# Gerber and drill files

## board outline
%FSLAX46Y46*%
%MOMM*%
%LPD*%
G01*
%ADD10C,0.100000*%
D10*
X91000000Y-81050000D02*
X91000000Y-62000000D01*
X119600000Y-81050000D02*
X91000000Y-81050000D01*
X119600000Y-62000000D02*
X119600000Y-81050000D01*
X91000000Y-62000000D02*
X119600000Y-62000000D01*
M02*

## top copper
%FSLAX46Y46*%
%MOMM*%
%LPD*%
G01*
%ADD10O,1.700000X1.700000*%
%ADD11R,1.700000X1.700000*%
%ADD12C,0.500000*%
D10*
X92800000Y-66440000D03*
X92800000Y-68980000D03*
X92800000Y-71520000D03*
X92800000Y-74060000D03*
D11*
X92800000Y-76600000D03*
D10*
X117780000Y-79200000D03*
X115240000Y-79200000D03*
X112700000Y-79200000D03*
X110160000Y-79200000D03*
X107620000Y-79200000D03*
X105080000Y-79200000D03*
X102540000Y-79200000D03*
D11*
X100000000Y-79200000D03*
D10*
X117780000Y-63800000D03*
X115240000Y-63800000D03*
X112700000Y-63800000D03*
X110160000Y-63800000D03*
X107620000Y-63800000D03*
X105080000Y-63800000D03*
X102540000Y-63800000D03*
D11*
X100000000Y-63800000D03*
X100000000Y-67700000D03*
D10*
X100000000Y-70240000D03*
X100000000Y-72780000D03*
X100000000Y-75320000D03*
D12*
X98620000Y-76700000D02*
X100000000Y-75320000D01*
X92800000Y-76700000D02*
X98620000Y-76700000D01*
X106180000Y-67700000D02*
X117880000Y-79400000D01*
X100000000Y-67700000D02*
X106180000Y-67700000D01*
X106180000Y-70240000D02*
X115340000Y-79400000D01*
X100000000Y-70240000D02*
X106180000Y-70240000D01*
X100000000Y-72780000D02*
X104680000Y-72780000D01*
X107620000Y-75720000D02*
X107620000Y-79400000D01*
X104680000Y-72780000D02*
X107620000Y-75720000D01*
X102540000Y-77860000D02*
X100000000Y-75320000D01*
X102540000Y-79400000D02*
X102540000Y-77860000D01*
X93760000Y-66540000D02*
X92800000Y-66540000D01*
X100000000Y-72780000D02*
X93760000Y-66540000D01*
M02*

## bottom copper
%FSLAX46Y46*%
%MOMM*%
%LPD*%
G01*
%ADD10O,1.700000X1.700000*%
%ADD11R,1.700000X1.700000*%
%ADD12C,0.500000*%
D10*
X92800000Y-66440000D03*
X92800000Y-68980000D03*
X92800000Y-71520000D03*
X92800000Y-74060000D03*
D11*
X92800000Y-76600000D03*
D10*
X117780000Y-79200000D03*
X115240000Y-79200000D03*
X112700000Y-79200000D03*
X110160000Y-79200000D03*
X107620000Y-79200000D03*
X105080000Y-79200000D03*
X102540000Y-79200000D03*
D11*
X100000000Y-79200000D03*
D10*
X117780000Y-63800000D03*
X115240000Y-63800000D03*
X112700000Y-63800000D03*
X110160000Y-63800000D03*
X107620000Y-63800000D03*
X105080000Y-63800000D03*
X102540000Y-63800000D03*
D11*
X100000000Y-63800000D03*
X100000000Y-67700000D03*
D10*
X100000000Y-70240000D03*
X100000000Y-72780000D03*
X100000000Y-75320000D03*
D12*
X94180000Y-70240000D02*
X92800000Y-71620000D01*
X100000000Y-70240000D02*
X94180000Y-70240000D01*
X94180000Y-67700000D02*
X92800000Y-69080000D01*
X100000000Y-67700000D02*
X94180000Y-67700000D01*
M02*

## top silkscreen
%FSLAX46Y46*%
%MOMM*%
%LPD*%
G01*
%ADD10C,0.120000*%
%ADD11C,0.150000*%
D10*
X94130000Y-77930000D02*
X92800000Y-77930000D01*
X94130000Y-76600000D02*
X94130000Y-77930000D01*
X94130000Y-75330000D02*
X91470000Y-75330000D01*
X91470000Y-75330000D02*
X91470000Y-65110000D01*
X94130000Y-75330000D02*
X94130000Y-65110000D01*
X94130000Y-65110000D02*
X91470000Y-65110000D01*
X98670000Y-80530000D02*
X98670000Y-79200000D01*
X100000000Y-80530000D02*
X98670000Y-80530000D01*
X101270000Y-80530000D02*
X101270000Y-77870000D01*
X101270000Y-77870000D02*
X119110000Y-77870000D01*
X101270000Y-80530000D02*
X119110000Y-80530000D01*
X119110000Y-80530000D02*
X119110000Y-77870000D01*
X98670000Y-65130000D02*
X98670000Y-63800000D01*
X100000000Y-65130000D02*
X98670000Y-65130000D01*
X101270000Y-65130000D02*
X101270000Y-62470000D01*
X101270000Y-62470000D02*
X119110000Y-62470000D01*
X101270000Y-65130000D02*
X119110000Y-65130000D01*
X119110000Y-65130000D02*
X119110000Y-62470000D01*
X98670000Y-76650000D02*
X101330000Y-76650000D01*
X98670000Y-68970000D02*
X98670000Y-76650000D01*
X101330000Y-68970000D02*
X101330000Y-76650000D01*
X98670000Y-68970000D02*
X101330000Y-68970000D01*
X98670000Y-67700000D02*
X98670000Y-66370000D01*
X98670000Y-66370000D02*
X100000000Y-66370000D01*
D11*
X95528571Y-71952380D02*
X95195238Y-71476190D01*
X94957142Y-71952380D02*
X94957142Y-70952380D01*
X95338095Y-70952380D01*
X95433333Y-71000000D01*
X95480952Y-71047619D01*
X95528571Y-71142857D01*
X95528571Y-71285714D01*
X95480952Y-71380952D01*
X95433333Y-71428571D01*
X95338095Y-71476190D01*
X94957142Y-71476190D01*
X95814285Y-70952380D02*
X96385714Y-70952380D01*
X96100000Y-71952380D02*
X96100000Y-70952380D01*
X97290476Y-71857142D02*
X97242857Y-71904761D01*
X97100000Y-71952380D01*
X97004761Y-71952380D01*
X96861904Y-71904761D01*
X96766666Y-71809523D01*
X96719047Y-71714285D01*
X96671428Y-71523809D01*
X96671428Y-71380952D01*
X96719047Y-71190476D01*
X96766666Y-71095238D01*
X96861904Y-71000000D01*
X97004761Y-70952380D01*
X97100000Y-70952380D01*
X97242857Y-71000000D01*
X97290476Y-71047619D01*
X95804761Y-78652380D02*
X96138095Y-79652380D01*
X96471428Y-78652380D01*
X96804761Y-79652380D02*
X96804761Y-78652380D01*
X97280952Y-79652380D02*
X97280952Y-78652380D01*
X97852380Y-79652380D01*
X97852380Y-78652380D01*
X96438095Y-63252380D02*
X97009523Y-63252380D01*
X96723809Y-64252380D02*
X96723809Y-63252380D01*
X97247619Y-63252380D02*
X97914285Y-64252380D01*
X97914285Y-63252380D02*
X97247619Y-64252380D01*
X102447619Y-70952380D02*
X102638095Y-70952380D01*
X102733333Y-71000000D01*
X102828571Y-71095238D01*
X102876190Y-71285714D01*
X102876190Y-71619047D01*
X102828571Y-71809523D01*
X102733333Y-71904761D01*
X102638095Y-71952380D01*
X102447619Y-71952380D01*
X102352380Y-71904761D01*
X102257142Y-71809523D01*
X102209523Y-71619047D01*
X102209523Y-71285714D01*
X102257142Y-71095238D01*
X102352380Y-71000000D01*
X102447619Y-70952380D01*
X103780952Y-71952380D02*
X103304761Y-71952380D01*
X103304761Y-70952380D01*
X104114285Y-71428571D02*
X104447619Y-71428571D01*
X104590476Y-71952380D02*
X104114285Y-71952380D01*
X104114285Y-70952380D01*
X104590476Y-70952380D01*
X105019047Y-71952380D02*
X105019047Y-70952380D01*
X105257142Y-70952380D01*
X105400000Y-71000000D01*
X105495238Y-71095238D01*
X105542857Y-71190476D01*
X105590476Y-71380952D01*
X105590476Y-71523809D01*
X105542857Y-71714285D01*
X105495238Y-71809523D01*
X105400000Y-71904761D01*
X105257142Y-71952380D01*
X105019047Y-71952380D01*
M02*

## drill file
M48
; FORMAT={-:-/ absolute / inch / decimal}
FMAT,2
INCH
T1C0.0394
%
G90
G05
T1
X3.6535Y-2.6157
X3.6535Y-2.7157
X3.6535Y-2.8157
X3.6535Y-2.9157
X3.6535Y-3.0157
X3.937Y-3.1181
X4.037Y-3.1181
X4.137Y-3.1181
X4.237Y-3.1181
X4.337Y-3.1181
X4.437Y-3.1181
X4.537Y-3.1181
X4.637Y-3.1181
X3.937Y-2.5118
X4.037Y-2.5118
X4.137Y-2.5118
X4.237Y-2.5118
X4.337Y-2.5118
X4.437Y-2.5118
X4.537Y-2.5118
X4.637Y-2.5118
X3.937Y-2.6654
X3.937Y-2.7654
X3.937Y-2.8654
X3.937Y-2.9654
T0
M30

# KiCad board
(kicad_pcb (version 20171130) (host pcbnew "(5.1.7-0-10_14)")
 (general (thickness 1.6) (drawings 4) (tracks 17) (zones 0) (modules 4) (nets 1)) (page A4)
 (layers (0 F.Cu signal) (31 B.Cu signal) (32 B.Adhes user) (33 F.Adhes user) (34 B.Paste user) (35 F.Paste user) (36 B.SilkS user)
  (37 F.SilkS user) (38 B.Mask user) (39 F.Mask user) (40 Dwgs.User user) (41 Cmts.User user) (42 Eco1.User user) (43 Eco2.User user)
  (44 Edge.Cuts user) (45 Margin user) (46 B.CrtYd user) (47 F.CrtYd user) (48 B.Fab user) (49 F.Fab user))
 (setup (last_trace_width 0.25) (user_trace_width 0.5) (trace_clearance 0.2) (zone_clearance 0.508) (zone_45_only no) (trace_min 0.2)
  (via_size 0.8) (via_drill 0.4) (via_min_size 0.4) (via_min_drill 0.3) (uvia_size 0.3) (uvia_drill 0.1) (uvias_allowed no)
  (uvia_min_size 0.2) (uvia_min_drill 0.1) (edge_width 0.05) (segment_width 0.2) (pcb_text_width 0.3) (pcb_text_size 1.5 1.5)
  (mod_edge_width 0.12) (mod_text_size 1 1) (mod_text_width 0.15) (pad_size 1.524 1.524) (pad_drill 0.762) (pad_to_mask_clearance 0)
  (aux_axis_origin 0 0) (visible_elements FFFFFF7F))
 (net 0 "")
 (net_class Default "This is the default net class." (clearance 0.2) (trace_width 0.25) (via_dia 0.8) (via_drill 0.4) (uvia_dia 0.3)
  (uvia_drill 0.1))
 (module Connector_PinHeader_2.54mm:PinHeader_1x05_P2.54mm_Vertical (layer F.Cu) (at 92.8 76.6 180)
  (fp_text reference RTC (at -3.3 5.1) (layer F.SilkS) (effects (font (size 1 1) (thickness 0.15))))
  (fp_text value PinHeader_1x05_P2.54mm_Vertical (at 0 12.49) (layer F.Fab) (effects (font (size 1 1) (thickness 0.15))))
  (fp_line (start -1.33 -1.33) (end 0 -1.33) (layer F.SilkS) (width 0.12))
  (fp_line (start -1.33 0) (end -1.33 -1.33) (layer F.SilkS) (width 0.12))
  (fp_line (start -1.33 1.27) (end 1.33 1.27) (layer F.SilkS) (width 0.12))
  (fp_line (start 1.33 1.27) (end 1.33 11.49) (layer F.SilkS) (width 0.12))
  (fp_line (start -1.33 1.27) (end -1.33 11.49) (layer F.SilkS) (width 0.12))
  (fp_line (start -1.33 11.49) (end 1.33 11.49) (layer F.SilkS) (width 0.12))
  (pad 5 thru_hole oval (at 0 10.16 180) (size 1.7 1.7) (drill 1) (layers *.Cu *.Mask))
  (pad 4 thru_hole oval (at 0 7.62 180) (size 1.7 1.7) (drill 1) (layers *.Cu *.Mask))
  (pad 3 thru_hole oval (at 0 5.08 180) (size 1.7 1.7) (drill 1) (layers *.Cu *.Mask))
  (pad 2 thru_hole oval (at 0 2.54 180) (size 1.7 1.7) (drill 1) (layers *.Cu *.Mask))
  (pad 1 thru_hole rect (at 0 0 180) (size 1.7 1.7) (drill 1) (layers *.Cu *.Mask)))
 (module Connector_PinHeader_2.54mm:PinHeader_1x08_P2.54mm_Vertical (layer F.Cu) (at 100 79.2 90)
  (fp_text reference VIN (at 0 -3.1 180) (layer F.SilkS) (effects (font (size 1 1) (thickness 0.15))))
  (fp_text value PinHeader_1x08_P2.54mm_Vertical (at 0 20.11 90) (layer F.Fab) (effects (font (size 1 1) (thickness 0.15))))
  (fp_line (start -1.33 -1.33) (end 0 -1.33) (layer F.SilkS) (width 0.12))
  (fp_line (start -1.33 0) (end -1.33 -1.33) (layer F.SilkS) (width 0.12))
  (fp_line (start -1.33 1.27) (end 1.33 1.27) (layer F.SilkS) (width 0.12))
  (fp_line (start 1.33 1.27) (end 1.33 19.11) (layer F.SilkS) (width 0.12))
  (fp_line (start -1.33 1.27) (end -1.33 19.11) (layer F.SilkS) (width 0.12))
  (fp_line (start -1.33 19.11) (end 1.33 19.11) (layer F.SilkS) (width 0.12))
  (pad 8 thru_hole oval (at 0 17.78 90) (size 1.7 1.7) (drill 1) (layers *.Cu *.Mask))
  (pad 7 thru_hole oval (at 0 15.24 90) (size 1.7 1.7) (drill 1) (layers *.Cu *.Mask))
  (pad 6 thru_hole oval (at 0 12.7 90) (size 1.7 1.7) (drill 1) (layers *.Cu *.Mask))
  (pad 5 thru_hole oval (at 0 10.16 90) (size 1.7 1.7) (drill 1) (layers *.Cu *.Mask))
  (pad 4 thru_hole oval (at 0 7.62 90) (size 1.7 1.7) (drill 1) (layers *.Cu *.Mask))
  (pad 3 thru_hole oval (at 0 5.08 90) (size 1.7 1.7) (drill 1) (layers *.Cu *.Mask))
  (pad 2 thru_hole oval (at 0 2.54 90) (size 1.7 1.7) (drill 1) (layers *.Cu *.Mask))
  (pad 1 thru_hole rect (at 0 0 90) (size 1.7 1.7) (drill 1) (layers *.Cu *.Mask)))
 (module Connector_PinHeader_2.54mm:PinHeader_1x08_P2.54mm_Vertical (layer F.Cu) (at 100 63.8 90)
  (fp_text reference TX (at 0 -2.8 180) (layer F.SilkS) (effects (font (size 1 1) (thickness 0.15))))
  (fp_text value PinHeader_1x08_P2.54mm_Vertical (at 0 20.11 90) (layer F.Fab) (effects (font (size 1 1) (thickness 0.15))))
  (fp_line (start -1.33 -1.33) (end 0 -1.33) (layer F.SilkS) (width 0.12))
  (fp_line (start -1.33 0) (end -1.33 -1.33) (layer F.SilkS) (width 0.12))
  (fp_line (start -1.33 1.27) (end 1.33 1.27) (layer F.SilkS) (width 0.12))
  (fp_line (start 1.33 1.27) (end 1.33 19.11) (layer F.SilkS) (width 0.12))
  (fp_line (start -1.33 1.27) (end -1.33 19.11) (layer F.SilkS) (width 0.12))
  (fp_line (start -1.33 19.11) (end 1.33 19.11) (layer F.SilkS) (width 0.12))
  (pad 8 thru_hole oval (at 0 17.78 90) (size 1.7 1.7) (drill 1) (layers *.Cu *.Mask))
  (pad 7 thru_hole oval (at 0 15.24 90) (size 1.7 1.7) (drill 1) (layers *.Cu *.Mask))
  (pad 6 thru_hole oval (at 0 12.7 90) (size 1.7 1.7) (drill 1) (layers *.Cu *.Mask))
  (pad 5 thru_hole oval (at 0 10.16 90) (size 1.7 1.7) (drill 1) (layers *.Cu *.Mask))
  (pad 4 thru_hole oval (at 0 7.62 90) (size 1.7 1.7) (drill 1) (layers *.Cu *.Mask))
  (pad 3 thru_hole oval (at 0 5.08 90) (size 1.7 1.7) (drill 1) (layers *.Cu *.Mask))
  (pad 2 thru_hole oval (at 0 2.54 90) (size 1.7 1.7) (drill 1) (layers *.Cu *.Mask))
  (pad 1 thru_hole rect (at 0 0 90) (size 1.7 1.7) (drill 1) (layers *.Cu *.Mask)))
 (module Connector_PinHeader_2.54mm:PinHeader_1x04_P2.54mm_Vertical (layer F.Cu) (at 100 67.7)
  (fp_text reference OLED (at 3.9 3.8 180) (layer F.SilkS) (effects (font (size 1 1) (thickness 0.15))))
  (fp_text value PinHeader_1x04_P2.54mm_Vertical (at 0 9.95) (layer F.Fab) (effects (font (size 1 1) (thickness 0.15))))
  (fp_line (start -1.33 8.95) (end 1.33 8.95) (layer F.SilkS) (width 0.12))
  (fp_line (start -1.33 1.27) (end -1.33 8.95) (layer F.SilkS) (width 0.12))
  (fp_line (start 1.33 1.27) (end 1.33 8.95) (layer F.SilkS) (width 0.12))
  (fp_line (start -1.33 1.27) (end 1.33 1.27) (layer F.SilkS) (width 0.12))
  (fp_line (start -1.33 0) (end -1.33 -1.33) (layer F.SilkS) (width 0.12))
  (fp_line (start -1.33 -1.33) (end 0 -1.33) (layer F.SilkS) (width 0.12))
  (pad 1 thru_hole rect (at 0 0) (size 1.7 1.7) (drill 1) (layers *.Cu *.Mask))
  (pad 2 thru_hole oval (at 0 2.54) (size 1.7 1.7) (drill 1) (layers *.Cu *.Mask))
  (pad 3 thru_hole oval (at 0 5.08) (size 1.7 1.7) (drill 1) (layers *.Cu *.Mask))
  (pad 4 thru_hole oval (at 0 7.62) (size 1.7 1.7) (drill 1) (layers *.Cu *.Mask)))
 (gr_line (start 91 81.05) (end 91 62) (layer Edge.Cuts) (width 0.1))
 (gr_line (start 119.6 81.05) (end 91 81.05) (layer Edge.Cuts) (width 0.1))
 (gr_line (start 119.6 62) (end 119.6 81.05) (layer Edge.Cuts) (width 0.1))
 (gr_line (start 91 62) (end 119.6 62) (layer Edge.Cuts) (width 0.1))
 (segment (start 98.62 76.7) (end 100 75.32) (width 0.5) (layer F.Cu) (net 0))
 (segment (start 92.8 76.7) (end 98.62 76.7) (width 0.5) (layer F.Cu) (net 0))
 (segment (start 106.18 67.7) (end 117.88 79.4) (width 0.5) (layer F.Cu) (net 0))
 (segment (start 100 67.7) (end 106.18 67.7) (width 0.5) (layer F.Cu) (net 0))
 (segment (start 106.18 70.24) (end 115.34 79.4) (width 0.5) (layer F.Cu) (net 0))
 (segment (start 100 70.24) (end 106.18 70.24) (width 0.5) (layer F.Cu) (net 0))
 (segment (start 94.18 70.24) (end 92.8 71.62) (width 0.5) (layer B.Cu) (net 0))
 (segment (start 100 70.24) (end 94.18 70.24) (width 0.5) (layer B.Cu) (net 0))
 (segment (start 100 72.78) (end 104.68 72.78) (width 0.5) (layer F.Cu) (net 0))
 (segment (start 107.62 75.72) (end 107.62 79.4) (width 0.5) (layer F.Cu) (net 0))
 (segment (start 104.68 72.78) (end 107.62 75.72) (width 0.5) (layer F.Cu) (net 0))
 (segment (start 102.54 77.86) (end 100 75.32) (width 0.5) (layer F.Cu) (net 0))
 (segment (start 102.54 79.4) (end 102.54 77.86) (width 0.5) (layer F.Cu) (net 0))
 (segment (start 94.18 67.7) (end 92.8 69.08) (width 0.5) (layer B.Cu) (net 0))
 (segment (start 100 67.7) (end 94.18 67.7) (width 0.5) (layer B.Cu) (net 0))
 (segment (start 93.76 66.54) (end 92.8 66.54) (width 0.5) (layer F.Cu) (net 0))
 (segment (start 100 72.78) (end 93.76 66.54) (width 0.5) (layer F.Cu) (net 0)))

